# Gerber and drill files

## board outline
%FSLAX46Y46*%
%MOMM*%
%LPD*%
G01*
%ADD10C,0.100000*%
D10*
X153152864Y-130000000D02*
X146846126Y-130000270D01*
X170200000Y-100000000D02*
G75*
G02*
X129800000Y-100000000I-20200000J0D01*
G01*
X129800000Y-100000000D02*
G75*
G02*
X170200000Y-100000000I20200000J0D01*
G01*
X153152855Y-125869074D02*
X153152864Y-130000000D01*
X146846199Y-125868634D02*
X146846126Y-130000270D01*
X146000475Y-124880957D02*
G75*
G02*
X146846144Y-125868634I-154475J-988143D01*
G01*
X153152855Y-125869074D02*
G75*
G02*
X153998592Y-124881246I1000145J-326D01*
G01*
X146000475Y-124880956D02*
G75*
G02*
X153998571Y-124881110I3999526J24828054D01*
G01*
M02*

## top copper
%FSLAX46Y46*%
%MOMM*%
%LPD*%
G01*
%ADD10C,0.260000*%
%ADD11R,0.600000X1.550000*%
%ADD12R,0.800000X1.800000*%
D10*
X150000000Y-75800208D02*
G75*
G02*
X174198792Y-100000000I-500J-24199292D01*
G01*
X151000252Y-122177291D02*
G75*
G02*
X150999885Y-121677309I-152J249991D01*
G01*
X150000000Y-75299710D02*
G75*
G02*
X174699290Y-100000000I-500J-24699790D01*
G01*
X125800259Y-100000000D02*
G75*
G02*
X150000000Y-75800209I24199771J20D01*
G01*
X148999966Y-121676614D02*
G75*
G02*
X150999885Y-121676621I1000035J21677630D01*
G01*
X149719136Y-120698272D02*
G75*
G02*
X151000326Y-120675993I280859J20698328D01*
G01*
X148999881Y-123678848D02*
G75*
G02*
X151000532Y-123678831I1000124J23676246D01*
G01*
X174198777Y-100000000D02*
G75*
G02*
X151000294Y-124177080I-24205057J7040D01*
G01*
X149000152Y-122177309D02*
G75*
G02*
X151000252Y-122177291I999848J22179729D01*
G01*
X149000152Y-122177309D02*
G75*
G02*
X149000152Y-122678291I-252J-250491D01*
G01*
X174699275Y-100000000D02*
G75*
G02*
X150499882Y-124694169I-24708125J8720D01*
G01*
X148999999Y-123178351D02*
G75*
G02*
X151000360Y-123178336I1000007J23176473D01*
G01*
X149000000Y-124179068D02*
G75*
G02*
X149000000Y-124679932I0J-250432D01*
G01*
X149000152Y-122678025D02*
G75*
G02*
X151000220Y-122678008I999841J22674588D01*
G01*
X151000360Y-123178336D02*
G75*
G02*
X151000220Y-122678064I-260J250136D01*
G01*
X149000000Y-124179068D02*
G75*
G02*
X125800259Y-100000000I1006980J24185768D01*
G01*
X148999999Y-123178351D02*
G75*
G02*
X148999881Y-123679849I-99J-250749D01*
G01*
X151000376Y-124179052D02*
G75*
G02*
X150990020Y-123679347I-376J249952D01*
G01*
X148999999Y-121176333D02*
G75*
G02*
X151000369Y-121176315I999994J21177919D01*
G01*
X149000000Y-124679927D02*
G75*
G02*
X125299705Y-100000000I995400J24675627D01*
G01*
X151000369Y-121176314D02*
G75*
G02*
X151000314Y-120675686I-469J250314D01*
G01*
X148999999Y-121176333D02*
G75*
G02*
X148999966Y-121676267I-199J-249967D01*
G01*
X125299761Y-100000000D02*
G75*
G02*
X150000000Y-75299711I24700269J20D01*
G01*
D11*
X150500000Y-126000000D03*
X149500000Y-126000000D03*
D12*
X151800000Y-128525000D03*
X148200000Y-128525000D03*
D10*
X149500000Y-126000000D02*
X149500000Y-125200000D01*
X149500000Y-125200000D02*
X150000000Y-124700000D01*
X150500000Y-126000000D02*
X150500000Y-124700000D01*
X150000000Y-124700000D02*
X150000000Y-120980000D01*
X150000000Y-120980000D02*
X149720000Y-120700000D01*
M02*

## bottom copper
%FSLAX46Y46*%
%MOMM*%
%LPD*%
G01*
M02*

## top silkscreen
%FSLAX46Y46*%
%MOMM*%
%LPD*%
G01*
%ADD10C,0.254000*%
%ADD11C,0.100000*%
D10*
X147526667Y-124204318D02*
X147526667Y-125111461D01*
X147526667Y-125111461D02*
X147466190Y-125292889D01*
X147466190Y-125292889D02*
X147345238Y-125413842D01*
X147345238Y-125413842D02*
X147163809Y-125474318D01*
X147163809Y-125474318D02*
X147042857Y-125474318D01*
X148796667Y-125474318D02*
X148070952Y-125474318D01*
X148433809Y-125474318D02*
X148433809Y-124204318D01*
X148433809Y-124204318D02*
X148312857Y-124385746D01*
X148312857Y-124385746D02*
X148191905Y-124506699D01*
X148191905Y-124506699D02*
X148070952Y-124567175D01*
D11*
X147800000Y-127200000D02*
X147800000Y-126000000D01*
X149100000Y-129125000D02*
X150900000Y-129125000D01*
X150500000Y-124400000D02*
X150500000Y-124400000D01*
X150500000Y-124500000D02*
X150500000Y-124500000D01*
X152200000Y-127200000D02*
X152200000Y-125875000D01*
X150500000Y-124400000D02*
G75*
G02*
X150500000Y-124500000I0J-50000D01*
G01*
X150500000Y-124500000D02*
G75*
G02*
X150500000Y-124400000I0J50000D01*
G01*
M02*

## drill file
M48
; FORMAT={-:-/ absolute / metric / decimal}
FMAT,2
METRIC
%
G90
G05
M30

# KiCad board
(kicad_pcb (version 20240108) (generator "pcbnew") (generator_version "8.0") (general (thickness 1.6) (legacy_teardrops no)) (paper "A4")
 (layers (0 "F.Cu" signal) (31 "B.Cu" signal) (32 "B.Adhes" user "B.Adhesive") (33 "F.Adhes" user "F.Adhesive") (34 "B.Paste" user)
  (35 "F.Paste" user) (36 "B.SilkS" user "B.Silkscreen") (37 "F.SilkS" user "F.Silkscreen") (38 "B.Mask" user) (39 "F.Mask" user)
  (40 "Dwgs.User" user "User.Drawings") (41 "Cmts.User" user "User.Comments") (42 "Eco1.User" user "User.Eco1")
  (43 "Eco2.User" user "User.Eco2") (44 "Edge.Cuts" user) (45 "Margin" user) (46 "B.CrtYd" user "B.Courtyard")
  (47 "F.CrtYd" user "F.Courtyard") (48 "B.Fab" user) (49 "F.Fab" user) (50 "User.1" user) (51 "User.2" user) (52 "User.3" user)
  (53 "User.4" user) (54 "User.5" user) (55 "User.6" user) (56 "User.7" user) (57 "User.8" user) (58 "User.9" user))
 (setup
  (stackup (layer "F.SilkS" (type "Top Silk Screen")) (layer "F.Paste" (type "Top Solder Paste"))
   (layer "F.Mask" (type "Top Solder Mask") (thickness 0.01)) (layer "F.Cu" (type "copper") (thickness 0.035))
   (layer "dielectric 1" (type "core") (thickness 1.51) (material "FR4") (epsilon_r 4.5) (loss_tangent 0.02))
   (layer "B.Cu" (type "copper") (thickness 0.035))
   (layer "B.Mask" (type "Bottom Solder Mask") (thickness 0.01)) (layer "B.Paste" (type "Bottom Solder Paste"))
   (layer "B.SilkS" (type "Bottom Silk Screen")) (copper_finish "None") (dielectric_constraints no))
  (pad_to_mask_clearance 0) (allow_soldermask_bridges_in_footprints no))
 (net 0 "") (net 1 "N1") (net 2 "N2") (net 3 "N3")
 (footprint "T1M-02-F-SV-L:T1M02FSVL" (layer "F.Cu") (at 150 127.5 180)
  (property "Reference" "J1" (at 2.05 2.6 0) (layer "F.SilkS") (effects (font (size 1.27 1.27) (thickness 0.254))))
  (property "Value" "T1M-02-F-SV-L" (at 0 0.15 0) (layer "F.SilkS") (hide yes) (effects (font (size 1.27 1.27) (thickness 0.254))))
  (fp_line (start 2.2 0.3) (end 2.2 1.5) (stroke (width 0.1) (type solid)) (layer "F.SilkS"))
  (fp_line (start 0.9 -1.625) (end -0.9 -1.625) (stroke (width 0.1) (type solid)) (layer "F.SilkS"))
  (fp_line (start -0.5 3.1) (end -0.5 3.1) (stroke (width 0.1) (type solid)) (layer "F.SilkS"))
  (fp_line (start -0.5 3) (end -0.5 3) (stroke (width 0.1) (type solid)) (layer "F.SilkS"))
  (fp_line (start -2.2 0.3) (end -2.2 1.625) (stroke (width 0.1) (type solid)) (layer "F.SilkS"))
  (fp_arc (start -0.5 3.1) (mid -0.55 3.05) (end -0.5 3) (stroke (width 0.1) (type solid)) (layer "F.SilkS"))
  (fp_arc (start -0.5 3) (mid -0.45 3.05) (end -0.5 3.1) (stroke (width 0.1) (type solid)) (layer "F.SilkS"))
  (pad "1" smd rect (at -0.5 1.5 180) (size 0.6 1.55) (layers "F.Cu" "F.Paste" "F.Mask") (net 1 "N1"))
  (pad "2" smd rect (at 0.5 1.5 180) (size 0.6 1.55) (layers "F.Cu" "F.Paste" "F.Mask") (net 1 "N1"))
  (pad "MP1" smd rect (at -1.8 -1.025 180) (size 0.8 1.8) (layers "F.Cu" "F.Paste" "F.Mask") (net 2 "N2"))
  (pad "MP2" smd rect (at 1.8 -1.025 180) (size 0.8 1.8) (layers "F.Cu" "F.Paste" "F.Mask") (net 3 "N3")))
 (gr_arc (start 150 75.800208) (mid 167.111329 82.888373) (end 174.198777 100) (stroke (width 0.26) (type solid)) (layer "F.Cu") (net 1))
 (gr_arc (start 151.000252 122.177291) (mid 150.750104 121.927509) (end 150.999885 121.677361) (stroke (width 0.26) (type solid))
  (layer "F.Cu") (net 1))
 (gr_arc (start 150 75.29971) (mid 167.465235 82.534468) (end 174.699275 100) (stroke (width 0.26) (type solid)) (layer "F.Cu") (net 1))
 (gr_arc (start 125.800259 100) (mid 132.888189 82.888174) (end 150 75.800208) (stroke (width 0.26) (type solid)) (layer "F.Cu") (net 1))
 (gr_arc (start 148.999966 121.676614) (mid 150.000077 78.298299) (end 150.999885 121.676621) (stroke (width 0.26) (type solid))
  (layer "F.Cu") (net 1))
 (gr_arc (start 149.719136 120.698272) (mid 149.640087 79.30284) (end 151.000326 120.675993) (stroke (width 0.26) (type solid))
  (layer "F.Cu") (net 1))
 (gr_arc (start 148.999881 123.678848) (mid 149.999803 76.305242) (end 151.000532 123.678831) (stroke (width 0.26) (type solid))
  (layer "F.Cu") (net 1))
 (gr_arc (start 174.198777 100) (mid 167.459097 116.751403) (end 151.000294 124.177077) (stroke (width 0.26) (type solid)) (layer "F.Cu")
  (net 1))
 (gr_arc (start 149.000152 122.177309) (mid 149.999802 77.795324) (end 151.000252 122.177291) (stroke (width 0.26) (type solid))
  (layer "F.Cu") (net 1))
 (gr_arc (start 149.000152 122.177309) (mid 149.250395 122.427771) (end 149.000152 122.678233) (stroke (width 0.26) (type solid))
  (layer "F.Cu") (net 1))
 (gr_arc (start 174.699275 100) (mid 167.638329 117.284877) (end 150.499882 124.694165) (stroke (width 0.26) (type solid)) (layer "F.Cu")
  (net 1))
 (gr_arc (start 148.999999 123.178351) (mid 149.999832 76.803841) (end 151.00036 123.178336) (stroke (width 0.26) (type solid))
  (layer "F.Cu") (net 1))
 (gr_arc (start 149 124.179068) (mid 149.25043 124.429498) (end 149 124.679928) (stroke (width 0.26) (type solid)) (layer "F.Cu") (net 1))
 (gr_arc (start 149.000152 122.678025) (mid 149.9998 77.306816) (end 151.00022 122.678008) (stroke (width 0.26) (type solid)) (layer "F.Cu")
  (net 1))
 (gr_arc (start 151.00036 123.178336) (mid 150.749897 122.928231) (end 151.00022 122.677986) (stroke (width 0.26) (type solid))
  (layer "F.Cu") (net 1))
 (gr_arc (start 149 124.179068) (mid 132.540168 116.752652) (end 125.800259 100) (stroke (width 0.26) (type solid)) (layer "F.Cu") (net 1))
 (gr_arc (start 148.999999 123.178351) (mid 149.250697 123.429167) (end 148.999881 123.679865) (stroke (width 0.26) (type solid))
  (layer "F.Cu") (net 1))
 (gr_arc (start 151.000376 124.179052) (mid 150.750132 123.93431) (end 150.990023 123.679413) (stroke (width 0.26) (type solid))
  (layer "F.Cu") (net 1))
 (gr_arc (start 148.999999 121.176333) (mid 149.999802 78.796899) (end 151.000369 121.176315) (stroke (width 0.26) (type solid))
  (layer "F.Cu") (net 1))
 (gr_arc (start 149 124.679927) (mid 132.182992 117.109688) (end 125.299761 100) (stroke (width 0.26) (type solid)) (layer "F.Cu") (net 1))
 (gr_arc (start 151.000369 121.176314) (mid 150.74962 120.926057) (end 151.000314 120.675746) (stroke (width 0.26) (type solid))
  (layer "F.Cu") (net 1))
 (gr_arc (start 148.999999 121.176333) (mid 149.249754 121.426338) (end 148.999966 121.676311) (stroke (width 0.26) (type solid))
  (layer "F.Cu") (net 1))
 (gr_arc (start 125.299761 100) (mid 132.534283 82.534269) (end 150 75.29971) (stroke (width 0.26) (type solid)) (layer "F.Cu") (net 1))
 (gr_line (start 153.152864 130) (end 146.846126 130.00027) (stroke (width 0.1) (type solid)) (layer "Edge.Cuts"))
 (gr_circle (center 150 100) (end 170.2 100) (stroke (width 0.1) (type solid)) (fill none) (layer "Edge.Cuts"))
 (gr_line (start 153.152855 125.869074) (end 153.152864 130) (stroke (width 0.1) (type solid)) (layer "Edge.Cuts"))
 (gr_line (start 146.846199 125.868634) (end 146.846126 130.00027) (stroke (width 0.1) (type solid)) (layer "Edge.Cuts"))
 (gr_arc (start 146.000475 124.880957) (mid 146.605735 125.218613) (end 146.846199 125.868634) (stroke (width 0.1) (type solid))
  (layer "Edge.Cuts"))
 (gr_arc (start 153.152855 125.869074) (mid 153.393264 125.218946) (end 153.998592 124.881245) (stroke (width 0.1) (type solid))
  (layer "Edge.Cuts"))
 (gr_arc (start 146.000475 124.880956) (mid 150.000485 74.904771) (end 153.998571 124.88111) (stroke (width 0.1) (type solid))
  (layer "Edge.Cuts"))
 (segment (start 149.5 126) (end 149.5 125.2) (width 0.26) (layer "F.Cu") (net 1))
 (segment (start 149.5 125.2) (end 150 124.7) (width 0.26) (layer "F.Cu") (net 1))
 (segment (start 150.5 126) (end 150.5 124.7) (width 0.26) (layer "F.Cu") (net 1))
 (segment (start 150 124.7) (end 150 120.98) (width 0.26) (layer "F.Cu") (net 1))
 (segment (start 150 120.98) (end 149.72 120.7) (width 0.26) (layer "F.Cu") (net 1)))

